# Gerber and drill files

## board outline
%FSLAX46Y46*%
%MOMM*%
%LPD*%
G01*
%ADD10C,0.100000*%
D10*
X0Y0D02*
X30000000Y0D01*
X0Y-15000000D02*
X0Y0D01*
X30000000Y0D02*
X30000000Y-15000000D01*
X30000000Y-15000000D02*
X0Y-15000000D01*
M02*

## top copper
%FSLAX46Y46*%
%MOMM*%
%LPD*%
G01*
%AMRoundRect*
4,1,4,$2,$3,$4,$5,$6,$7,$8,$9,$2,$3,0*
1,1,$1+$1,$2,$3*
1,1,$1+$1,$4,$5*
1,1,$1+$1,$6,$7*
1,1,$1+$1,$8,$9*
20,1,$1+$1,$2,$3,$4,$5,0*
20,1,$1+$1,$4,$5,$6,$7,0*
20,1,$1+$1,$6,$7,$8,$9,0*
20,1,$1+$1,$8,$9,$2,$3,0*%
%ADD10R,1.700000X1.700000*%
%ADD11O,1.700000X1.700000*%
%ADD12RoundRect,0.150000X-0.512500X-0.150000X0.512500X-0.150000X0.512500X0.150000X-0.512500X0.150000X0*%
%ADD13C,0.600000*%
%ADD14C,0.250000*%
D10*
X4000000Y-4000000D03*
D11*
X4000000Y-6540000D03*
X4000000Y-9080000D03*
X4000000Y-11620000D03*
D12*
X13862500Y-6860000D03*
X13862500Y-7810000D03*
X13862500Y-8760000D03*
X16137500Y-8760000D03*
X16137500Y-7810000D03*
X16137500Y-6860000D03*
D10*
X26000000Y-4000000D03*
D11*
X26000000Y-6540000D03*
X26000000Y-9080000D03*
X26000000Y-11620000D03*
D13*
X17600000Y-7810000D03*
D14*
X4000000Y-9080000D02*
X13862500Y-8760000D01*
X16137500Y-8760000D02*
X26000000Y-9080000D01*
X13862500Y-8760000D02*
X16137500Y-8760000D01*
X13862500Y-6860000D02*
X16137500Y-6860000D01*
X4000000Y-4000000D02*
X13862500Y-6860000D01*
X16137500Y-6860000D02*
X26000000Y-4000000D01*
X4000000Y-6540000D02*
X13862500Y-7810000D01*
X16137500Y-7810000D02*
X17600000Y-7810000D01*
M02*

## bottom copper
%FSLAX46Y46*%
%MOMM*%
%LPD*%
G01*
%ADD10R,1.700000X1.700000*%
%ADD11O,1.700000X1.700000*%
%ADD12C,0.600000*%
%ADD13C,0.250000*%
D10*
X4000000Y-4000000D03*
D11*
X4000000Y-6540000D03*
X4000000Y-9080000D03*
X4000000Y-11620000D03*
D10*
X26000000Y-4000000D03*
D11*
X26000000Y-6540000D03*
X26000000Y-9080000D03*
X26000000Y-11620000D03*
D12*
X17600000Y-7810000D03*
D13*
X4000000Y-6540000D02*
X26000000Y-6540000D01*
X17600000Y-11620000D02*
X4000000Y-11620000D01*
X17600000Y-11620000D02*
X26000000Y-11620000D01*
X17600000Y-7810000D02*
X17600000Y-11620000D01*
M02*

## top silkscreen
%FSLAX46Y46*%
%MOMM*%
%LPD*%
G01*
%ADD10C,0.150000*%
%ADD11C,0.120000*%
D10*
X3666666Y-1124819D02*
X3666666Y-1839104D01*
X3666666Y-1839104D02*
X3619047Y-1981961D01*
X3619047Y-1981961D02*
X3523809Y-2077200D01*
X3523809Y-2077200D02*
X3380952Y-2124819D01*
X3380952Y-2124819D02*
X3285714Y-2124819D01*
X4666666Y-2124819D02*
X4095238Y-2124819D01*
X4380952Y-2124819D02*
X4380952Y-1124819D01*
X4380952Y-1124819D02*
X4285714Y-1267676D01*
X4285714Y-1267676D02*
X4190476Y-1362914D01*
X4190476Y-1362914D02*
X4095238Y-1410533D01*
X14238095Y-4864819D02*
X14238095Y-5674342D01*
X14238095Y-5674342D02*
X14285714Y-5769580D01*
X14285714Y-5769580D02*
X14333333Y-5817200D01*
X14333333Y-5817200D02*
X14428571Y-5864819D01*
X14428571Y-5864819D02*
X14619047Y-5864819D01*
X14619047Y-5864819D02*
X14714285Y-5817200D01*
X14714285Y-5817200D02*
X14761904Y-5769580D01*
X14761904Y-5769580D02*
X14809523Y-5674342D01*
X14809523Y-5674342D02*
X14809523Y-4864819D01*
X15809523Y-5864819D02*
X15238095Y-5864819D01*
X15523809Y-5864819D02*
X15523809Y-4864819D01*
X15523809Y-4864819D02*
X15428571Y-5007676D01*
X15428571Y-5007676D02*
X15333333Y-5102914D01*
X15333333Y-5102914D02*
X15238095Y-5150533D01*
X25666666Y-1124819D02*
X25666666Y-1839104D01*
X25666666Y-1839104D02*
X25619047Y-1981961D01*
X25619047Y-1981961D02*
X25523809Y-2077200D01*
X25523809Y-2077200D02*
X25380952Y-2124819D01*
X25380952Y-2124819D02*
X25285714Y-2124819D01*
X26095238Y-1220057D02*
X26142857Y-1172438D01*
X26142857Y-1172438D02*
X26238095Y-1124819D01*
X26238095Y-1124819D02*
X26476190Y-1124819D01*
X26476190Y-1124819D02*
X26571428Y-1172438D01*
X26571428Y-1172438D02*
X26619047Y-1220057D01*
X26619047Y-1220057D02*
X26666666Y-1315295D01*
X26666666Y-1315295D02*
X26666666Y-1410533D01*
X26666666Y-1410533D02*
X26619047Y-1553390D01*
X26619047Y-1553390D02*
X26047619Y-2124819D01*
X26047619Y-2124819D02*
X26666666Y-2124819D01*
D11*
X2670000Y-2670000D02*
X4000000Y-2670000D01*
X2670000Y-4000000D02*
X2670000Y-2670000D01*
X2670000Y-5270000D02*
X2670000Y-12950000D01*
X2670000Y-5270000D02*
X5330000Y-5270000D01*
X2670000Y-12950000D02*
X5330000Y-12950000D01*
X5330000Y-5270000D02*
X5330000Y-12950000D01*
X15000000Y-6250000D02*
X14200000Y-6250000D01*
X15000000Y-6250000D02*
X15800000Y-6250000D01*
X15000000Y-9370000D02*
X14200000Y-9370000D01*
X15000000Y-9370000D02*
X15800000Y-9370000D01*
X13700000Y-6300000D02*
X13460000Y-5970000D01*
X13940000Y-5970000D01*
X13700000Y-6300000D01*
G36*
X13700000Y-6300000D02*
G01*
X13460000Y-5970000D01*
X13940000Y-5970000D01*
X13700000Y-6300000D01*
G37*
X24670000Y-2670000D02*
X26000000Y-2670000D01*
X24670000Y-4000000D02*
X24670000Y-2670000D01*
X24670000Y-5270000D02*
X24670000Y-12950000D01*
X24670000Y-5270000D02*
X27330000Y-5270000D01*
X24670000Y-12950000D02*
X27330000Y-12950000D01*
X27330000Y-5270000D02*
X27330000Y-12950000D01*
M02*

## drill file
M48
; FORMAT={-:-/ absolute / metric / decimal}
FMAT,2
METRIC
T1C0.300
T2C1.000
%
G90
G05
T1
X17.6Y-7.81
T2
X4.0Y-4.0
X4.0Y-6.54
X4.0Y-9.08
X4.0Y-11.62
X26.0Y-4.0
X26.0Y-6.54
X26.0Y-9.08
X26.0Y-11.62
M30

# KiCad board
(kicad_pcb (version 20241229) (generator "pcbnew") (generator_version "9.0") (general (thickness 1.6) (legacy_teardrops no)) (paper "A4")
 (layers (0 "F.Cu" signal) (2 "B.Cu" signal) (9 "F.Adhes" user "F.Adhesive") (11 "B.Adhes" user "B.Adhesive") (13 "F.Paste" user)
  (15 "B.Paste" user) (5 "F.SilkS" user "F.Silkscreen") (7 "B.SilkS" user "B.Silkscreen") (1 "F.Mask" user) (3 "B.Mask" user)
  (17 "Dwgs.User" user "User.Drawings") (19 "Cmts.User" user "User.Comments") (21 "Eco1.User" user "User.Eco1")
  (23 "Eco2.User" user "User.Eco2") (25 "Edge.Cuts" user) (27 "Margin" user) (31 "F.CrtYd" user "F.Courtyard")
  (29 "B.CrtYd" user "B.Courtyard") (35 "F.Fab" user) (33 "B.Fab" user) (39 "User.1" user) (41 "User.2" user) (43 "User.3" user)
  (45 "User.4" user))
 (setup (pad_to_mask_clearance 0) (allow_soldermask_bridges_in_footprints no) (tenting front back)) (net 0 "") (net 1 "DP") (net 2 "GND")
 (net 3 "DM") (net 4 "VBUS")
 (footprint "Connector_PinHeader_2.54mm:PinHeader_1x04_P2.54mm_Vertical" (layer "F.Cu") (at 4 4)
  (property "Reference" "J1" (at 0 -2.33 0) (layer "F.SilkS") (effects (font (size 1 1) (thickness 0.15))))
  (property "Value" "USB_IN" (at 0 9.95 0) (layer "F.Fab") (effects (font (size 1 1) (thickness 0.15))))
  (fp_line (start -1.33 -1.33) (end 0 -1.33) (stroke (width 0.12) (type solid)) (layer "F.SilkS"))
  (fp_line (start -1.33 0) (end -1.33 -1.33) (stroke (width 0.12) (type solid)) (layer "F.SilkS"))
  (fp_line (start -1.33 1.27) (end -1.33 8.95) (stroke (width 0.12) (type solid)) (layer "F.SilkS"))
  (fp_line (start -1.33 1.27) (end 1.33 1.27) (stroke (width 0.12) (type solid)) (layer "F.SilkS"))
  (fp_line (start -1.33 8.95) (end 1.33 8.95) (stroke (width 0.12) (type solid)) (layer "F.SilkS"))
  (fp_line (start 1.33 1.27) (end 1.33 8.95) (stroke (width 0.12) (type solid)) (layer "F.SilkS"))
  (pad "1" thru_hole rect (at 0 0) (size 1.7 1.7) (drill 1) (layers "*.Cu" "*.Mask") (remove_unused_layers no) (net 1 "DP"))
  (pad "2" thru_hole oval (at 0 2.54) (size 1.7 1.7) (drill 1) (layers "*.Cu" "*.Mask") (remove_unused_layers no) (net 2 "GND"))
  (pad "3" thru_hole oval (at 0 5.08) (size 1.7 1.7) (drill 1) (layers "*.Cu" "*.Mask") (remove_unused_layers no) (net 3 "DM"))
  (pad "4" thru_hole oval (at 0 7.62) (size 1.7 1.7) (drill 1) (layers "*.Cu" "*.Mask") (remove_unused_layers no) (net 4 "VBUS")))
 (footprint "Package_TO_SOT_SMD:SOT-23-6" (layer "F.Cu") (at 15 7.81)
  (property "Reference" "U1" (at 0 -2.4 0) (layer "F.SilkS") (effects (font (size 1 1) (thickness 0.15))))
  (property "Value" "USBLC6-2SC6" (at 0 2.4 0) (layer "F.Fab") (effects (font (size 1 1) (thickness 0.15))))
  (fp_line (start 0 -1.56) (end -0.8 -1.56) (stroke (width 0.12) (type solid)) (layer "F.SilkS"))
  (fp_line (start 0 -1.56) (end 0.8 -1.56) (stroke (width 0.12) (type solid)) (layer "F.SilkS"))
  (fp_line (start 0 1.56) (end -0.8 1.56) (stroke (width 0.12) (type solid)) (layer "F.SilkS"))
  (fp_line (start 0 1.56) (end 0.8 1.56) (stroke (width 0.12) (type solid)) (layer "F.SilkS"))
  (fp_poly
   (pts (xy -1.3 -1.51) (xy -1.54 -1.84) (xy -1.06 -1.84) (xy -1.3 -1.51)) (stroke (width 0.12) (type solid)) (fill yes) (layer "F.SilkS"))
  (pad "1" smd roundrect (at -1.1375 -0.95) (size 1.325 0.6) (layers "F.Cu" "F.Mask" "F.Paste") (roundrect_rratio 0.25) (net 1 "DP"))
  (pad "2" smd roundrect (at -1.1375 0) (size 1.325 0.6) (layers "F.Cu" "F.Mask" "F.Paste") (roundrect_rratio 0.25) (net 2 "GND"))
  (pad "3" smd roundrect (at -1.1375 0.95) (size 1.325 0.6) (layers "F.Cu" "F.Mask" "F.Paste") (roundrect_rratio 0.25) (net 3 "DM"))
  (pad "4" smd roundrect (at 1.1375 0.95) (size 1.325 0.6) (layers "F.Cu" "F.Mask" "F.Paste") (roundrect_rratio 0.25) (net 3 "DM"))
  (pad "5" smd roundrect (at 1.1375 0) (size 1.325 0.6) (layers "F.Cu" "F.Mask" "F.Paste") (roundrect_rratio 0.25) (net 4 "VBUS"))
  (pad "6" smd roundrect (at 1.1375 -0.95) (size 1.325 0.6) (layers "F.Cu" "F.Mask" "F.Paste") (roundrect_rratio 0.25) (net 1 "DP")))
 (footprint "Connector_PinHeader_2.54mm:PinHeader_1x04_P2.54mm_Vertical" (layer "F.Cu") (at 26 4)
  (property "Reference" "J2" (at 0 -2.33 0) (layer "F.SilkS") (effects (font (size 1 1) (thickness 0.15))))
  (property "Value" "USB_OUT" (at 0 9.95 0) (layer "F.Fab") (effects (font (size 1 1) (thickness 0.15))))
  (fp_line (start -1.33 -1.33) (end 0 -1.33) (stroke (width 0.12) (type solid)) (layer "F.SilkS"))
  (fp_line (start -1.33 0) (end -1.33 -1.33) (stroke (width 0.12) (type solid)) (layer "F.SilkS"))
  (fp_line (start -1.33 1.27) (end -1.33 8.95) (stroke (width 0.12) (type solid)) (layer "F.SilkS"))
  (fp_line (start -1.33 1.27) (end 1.33 1.27) (stroke (width 0.12) (type solid)) (layer "F.SilkS"))
  (fp_line (start -1.33 8.95) (end 1.33 8.95) (stroke (width 0.12) (type solid)) (layer "F.SilkS"))
  (fp_line (start 1.33 1.27) (end 1.33 8.95) (stroke (width 0.12) (type solid)) (layer "F.SilkS"))
  (pad "1" thru_hole rect (at 0 0) (size 1.7 1.7) (drill 1) (layers "*.Cu" "*.Mask") (remove_unused_layers no) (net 1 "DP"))
  (pad "2" thru_hole oval (at 0 2.54) (size 1.7 1.7) (drill 1) (layers "*.Cu" "*.Mask") (remove_unused_layers no) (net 2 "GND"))
  (pad "3" thru_hole oval (at 0 5.08) (size 1.7 1.7) (drill 1) (layers "*.Cu" "*.Mask") (remove_unused_layers no) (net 3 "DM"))
  (pad "4" thru_hole oval (at 0 7.62) (size 1.7 1.7) (drill 1) (layers "*.Cu" "*.Mask") (remove_unused_layers no) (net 4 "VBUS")))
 (gr_line (start 0 0) (end 30 0) (stroke (width 0.1) (type default)) (layer "Edge.Cuts"))
 (gr_line (start 0 15) (end 0 0) (stroke (width 0.1) (type default)) (layer "Edge.Cuts"))
 (gr_line (start 30 0) (end 30 15) (stroke (width 0.1) (type default)) (layer "Edge.Cuts"))
 (gr_line (start 30 15) (end 0 15) (stroke (width 0.1) (type default)) (layer "Edge.Cuts"))
 (segment (start 4 9.08) (end 13.8625 8.76) (width 0.25) (layer "F.Cu") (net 3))
 (segment (start 16.1375 8.76) (end 26 9.08) (width 0.25) (layer "F.Cu") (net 3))
 (segment (start 13.8625 8.76) (end 16.1375 8.76) (width 0.25) (layer "F.Cu") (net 3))
 (segment (start 13.8625 6.86) (end 16.1375 6.86) (width 0.25) (layer "F.Cu") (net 1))
 (segment (start 4 4) (end 13.8625 6.86) (width 0.25) (layer "F.Cu") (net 1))
 (segment (start 16.1375 6.86) (end 26 4) (width 0.25) (layer "F.Cu") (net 1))
 (segment (start 4 6.54) (end 13.8625 7.81) (width 0.25) (layer "F.Cu") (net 2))
 (segment (start 4 6.54) (end 26 6.54) (width 0.25) (layer "B.Cu") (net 2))
 (segment (start 16.1375 7.81) (end 17.6 7.81) (width 0.25) (layer "F.Cu") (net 4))
 (via (at 17.6 7.81) (size 0.6) (drill 0.3) (layers "F.Cu" "B.Cu") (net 4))
 (segment (start 17.6 11.62) (end 4 11.62) (width 0.25) (layer "B.Cu") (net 4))
 (segment (start 17.6 11.62) (end 26 11.62) (width 0.25) (layer "B.Cu") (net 4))
 (segment (start 17.6 7.81) (end 17.6 11.62) (width 0.25) (layer "B.Cu") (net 4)))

